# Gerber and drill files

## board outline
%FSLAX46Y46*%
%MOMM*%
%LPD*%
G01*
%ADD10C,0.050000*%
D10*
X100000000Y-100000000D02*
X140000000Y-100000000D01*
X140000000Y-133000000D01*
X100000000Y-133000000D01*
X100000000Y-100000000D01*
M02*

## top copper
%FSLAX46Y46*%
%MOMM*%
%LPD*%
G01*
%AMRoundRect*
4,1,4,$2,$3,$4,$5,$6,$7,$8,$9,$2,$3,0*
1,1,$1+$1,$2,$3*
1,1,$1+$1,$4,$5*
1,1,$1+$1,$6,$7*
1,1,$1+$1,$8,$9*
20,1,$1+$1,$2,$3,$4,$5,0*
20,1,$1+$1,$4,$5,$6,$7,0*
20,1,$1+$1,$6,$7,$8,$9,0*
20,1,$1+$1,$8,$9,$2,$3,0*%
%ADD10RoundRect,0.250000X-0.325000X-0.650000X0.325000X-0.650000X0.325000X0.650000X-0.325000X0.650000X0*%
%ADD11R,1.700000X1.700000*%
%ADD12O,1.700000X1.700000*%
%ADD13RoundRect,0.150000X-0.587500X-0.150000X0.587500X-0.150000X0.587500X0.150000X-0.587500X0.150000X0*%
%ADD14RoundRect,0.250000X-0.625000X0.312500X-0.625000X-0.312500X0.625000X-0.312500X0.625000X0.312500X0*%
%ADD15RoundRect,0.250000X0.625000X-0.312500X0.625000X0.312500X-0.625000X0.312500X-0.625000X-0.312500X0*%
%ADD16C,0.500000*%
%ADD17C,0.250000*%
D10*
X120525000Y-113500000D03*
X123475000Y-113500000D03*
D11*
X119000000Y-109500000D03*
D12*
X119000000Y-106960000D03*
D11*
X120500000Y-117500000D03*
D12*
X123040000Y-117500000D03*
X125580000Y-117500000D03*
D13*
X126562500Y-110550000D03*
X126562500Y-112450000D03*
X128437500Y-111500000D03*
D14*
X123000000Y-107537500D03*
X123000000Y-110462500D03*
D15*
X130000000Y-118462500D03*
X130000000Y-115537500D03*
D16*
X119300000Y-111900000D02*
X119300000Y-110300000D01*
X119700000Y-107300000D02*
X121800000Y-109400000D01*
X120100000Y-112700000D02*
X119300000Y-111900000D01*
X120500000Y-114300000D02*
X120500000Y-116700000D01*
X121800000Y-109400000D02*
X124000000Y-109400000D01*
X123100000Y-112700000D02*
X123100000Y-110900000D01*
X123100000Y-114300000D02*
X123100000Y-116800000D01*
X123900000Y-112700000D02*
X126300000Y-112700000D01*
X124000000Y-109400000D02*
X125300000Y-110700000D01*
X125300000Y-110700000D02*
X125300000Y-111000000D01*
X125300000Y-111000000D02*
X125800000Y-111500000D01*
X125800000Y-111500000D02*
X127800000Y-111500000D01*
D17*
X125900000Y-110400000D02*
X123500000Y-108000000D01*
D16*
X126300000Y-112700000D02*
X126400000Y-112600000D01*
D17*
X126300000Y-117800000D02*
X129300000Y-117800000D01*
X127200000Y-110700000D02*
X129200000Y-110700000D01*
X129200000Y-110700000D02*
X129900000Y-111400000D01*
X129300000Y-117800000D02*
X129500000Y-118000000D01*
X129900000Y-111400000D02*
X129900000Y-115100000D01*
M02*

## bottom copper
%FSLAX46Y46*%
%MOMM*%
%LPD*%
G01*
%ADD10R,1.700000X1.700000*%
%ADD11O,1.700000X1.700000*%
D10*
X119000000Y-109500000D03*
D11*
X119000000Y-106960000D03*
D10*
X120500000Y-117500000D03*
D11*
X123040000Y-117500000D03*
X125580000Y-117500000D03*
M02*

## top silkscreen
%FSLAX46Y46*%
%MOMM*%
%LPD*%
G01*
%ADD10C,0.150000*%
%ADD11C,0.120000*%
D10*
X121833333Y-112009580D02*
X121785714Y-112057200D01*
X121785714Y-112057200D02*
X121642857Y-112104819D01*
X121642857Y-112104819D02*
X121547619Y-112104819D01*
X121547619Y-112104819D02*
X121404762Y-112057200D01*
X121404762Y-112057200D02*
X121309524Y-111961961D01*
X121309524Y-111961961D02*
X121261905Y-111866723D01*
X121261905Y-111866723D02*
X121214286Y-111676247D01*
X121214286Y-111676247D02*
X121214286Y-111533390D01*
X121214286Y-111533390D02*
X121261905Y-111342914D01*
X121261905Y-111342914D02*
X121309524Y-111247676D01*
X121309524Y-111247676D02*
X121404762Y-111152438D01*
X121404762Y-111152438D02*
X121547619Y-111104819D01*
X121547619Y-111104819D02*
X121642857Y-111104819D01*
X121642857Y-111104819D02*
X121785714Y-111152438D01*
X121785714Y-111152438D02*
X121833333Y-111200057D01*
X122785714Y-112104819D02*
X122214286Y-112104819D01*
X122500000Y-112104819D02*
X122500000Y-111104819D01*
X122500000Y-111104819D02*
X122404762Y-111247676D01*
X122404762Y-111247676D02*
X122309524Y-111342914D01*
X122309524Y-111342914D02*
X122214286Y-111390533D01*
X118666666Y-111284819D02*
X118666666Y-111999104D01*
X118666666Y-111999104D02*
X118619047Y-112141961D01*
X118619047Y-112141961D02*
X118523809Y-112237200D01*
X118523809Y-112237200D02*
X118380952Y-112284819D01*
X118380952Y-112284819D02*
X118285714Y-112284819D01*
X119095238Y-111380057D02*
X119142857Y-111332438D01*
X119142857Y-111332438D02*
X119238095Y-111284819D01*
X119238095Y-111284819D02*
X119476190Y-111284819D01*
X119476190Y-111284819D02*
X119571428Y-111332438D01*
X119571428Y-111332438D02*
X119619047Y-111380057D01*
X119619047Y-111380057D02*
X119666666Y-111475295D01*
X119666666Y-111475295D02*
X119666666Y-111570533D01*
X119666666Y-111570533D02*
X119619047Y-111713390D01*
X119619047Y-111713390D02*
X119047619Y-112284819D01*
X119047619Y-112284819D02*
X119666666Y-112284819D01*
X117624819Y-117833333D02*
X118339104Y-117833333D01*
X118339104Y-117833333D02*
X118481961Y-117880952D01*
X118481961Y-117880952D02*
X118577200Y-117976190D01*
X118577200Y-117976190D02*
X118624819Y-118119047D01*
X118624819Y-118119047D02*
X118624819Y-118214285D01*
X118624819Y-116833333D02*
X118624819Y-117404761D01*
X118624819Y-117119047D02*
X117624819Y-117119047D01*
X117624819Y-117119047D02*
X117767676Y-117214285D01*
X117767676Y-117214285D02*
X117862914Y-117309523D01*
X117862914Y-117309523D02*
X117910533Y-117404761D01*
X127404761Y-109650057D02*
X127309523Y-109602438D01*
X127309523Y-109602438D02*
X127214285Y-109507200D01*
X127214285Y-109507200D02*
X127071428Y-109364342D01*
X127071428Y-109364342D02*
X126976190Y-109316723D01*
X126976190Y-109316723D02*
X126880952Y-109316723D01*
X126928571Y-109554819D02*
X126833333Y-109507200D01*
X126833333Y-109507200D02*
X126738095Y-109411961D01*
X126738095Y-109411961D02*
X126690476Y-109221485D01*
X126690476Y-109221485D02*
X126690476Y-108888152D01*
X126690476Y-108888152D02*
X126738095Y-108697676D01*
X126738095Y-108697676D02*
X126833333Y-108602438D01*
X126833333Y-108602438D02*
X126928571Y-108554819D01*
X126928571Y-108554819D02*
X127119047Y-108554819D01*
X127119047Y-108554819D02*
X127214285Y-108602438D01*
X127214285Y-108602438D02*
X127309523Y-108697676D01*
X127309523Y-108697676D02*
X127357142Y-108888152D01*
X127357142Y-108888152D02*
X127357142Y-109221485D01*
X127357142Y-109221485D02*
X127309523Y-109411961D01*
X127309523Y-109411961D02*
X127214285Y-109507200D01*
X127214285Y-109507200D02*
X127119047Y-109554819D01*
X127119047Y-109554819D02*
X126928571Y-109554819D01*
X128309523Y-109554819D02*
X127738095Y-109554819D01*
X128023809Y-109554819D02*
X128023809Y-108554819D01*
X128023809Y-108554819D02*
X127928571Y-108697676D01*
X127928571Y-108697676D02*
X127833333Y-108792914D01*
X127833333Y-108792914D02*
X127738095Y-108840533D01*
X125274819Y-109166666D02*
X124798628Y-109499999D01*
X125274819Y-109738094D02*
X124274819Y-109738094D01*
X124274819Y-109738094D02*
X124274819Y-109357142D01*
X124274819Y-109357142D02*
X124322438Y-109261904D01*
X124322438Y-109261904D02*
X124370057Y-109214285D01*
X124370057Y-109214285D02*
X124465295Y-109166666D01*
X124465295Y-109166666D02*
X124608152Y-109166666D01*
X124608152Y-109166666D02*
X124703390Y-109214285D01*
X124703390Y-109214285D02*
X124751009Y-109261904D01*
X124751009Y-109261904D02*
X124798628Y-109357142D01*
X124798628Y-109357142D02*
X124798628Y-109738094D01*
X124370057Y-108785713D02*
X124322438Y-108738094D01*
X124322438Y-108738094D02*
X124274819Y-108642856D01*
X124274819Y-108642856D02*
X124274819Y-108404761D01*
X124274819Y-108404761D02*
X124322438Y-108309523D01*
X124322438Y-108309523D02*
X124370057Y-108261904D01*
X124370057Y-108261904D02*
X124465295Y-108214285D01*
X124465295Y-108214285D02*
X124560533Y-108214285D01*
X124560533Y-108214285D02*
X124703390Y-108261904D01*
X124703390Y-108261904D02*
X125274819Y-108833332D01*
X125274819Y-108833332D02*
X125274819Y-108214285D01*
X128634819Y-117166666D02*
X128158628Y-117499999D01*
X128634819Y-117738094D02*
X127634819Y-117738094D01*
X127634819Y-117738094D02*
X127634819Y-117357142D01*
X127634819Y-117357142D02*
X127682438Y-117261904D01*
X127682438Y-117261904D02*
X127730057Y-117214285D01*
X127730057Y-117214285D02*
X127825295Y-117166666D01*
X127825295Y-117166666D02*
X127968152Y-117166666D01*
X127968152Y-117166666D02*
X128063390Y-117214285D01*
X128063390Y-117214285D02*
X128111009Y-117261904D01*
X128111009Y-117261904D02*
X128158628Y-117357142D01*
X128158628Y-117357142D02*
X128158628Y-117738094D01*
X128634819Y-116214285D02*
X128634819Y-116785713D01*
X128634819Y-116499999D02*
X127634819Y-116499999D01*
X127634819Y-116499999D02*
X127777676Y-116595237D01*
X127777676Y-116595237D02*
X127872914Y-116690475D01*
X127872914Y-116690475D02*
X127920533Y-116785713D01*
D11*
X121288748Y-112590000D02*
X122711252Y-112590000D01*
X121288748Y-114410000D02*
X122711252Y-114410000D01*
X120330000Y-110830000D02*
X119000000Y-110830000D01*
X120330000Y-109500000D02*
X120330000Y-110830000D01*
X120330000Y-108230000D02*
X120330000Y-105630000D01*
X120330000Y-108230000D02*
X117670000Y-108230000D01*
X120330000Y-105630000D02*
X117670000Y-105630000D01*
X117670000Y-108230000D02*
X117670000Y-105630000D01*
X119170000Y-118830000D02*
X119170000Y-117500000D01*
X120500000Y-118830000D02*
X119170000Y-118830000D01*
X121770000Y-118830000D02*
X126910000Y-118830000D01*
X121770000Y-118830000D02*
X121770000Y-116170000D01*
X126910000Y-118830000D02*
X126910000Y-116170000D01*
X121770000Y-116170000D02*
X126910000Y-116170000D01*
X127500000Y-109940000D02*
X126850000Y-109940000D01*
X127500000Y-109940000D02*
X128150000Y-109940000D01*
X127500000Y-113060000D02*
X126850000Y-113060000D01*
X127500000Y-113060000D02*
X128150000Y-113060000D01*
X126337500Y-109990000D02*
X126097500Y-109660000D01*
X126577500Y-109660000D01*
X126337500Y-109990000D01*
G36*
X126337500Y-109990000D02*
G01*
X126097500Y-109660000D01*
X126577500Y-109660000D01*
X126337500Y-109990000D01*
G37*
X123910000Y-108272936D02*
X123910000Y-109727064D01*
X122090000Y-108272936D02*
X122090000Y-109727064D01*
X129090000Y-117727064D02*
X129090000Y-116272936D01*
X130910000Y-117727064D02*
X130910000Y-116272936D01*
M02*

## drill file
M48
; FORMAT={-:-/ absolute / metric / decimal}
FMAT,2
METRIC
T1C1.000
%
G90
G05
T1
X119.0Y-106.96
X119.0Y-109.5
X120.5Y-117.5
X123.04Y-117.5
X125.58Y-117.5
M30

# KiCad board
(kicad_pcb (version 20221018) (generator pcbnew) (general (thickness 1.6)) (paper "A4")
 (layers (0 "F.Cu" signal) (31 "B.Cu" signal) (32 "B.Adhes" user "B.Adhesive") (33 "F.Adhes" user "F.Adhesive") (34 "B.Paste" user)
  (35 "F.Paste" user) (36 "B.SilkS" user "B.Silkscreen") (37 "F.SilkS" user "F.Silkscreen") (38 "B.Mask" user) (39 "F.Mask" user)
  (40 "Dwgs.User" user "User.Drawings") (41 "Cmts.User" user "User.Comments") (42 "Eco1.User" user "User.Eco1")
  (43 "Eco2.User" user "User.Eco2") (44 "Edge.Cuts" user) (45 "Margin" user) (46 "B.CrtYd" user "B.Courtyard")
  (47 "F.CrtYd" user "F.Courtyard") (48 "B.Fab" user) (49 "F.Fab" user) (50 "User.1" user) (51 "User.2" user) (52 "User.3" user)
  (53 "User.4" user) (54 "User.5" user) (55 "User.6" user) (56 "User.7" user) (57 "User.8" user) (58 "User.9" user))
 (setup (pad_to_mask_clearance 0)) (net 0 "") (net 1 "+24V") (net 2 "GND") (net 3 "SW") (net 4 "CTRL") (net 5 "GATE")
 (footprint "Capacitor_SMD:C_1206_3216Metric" (layer "F.Cu") (at 122 113.5)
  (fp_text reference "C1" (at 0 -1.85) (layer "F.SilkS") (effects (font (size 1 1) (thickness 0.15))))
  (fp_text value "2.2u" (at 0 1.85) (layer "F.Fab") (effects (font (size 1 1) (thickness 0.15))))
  (fp_line (start -0.711252 -0.91) (end 0.711252 -0.91) (stroke (width 0.12) (type solid)) (layer "F.SilkS"))
  (fp_line (start -0.711252 0.91) (end 0.711252 0.91) (stroke (width 0.12) (type solid)) (layer "F.SilkS"))
  (pad "1" smd roundrect (at -1.475 0) (size 1.15 1.8) (layers "F.Cu" "F.Paste" "F.Mask") (roundrect_rratio 0.217391) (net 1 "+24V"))
  (pad "2" smd roundrect (at 1.475 0) (size 1.15 1.8) (layers "F.Cu" "F.Paste" "F.Mask") (roundrect_rratio 0.217391) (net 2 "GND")))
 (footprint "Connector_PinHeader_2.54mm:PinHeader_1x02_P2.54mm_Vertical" (layer "F.Cu") (at 119 109.5 180)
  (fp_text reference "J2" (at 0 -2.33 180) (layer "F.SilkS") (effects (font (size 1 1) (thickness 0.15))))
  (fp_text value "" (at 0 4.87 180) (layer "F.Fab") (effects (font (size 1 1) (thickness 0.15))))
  (fp_line (start -1.33 -1.33) (end 0 -1.33) (stroke (width 0.12) (type solid)) (layer "F.SilkS"))
  (fp_line (start -1.33 0) (end -1.33 -1.33) (stroke (width 0.12) (type solid)) (layer "F.SilkS"))
  (fp_line (start -1.33 1.27) (end -1.33 3.87) (stroke (width 0.12) (type solid)) (layer "F.SilkS"))
  (fp_line (start -1.33 1.27) (end 1.33 1.27) (stroke (width 0.12) (type solid)) (layer "F.SilkS"))
  (fp_line (start -1.33 3.87) (end 1.33 3.87) (stroke (width 0.12) (type solid)) (layer "F.SilkS"))
  (fp_line (start 1.33 1.27) (end 1.33 3.87) (stroke (width 0.12) (type solid)) (layer "F.SilkS"))
  (pad "1" thru_hole rect (at 0 0 180) (size 1.7 1.7) (drill 1) (layers "*.Cu" "*.Mask") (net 1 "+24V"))
  (pad "2" thru_hole oval (at 0 2.54 180) (size 1.7 1.7) (drill 1) (layers "*.Cu" "*.Mask") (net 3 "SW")))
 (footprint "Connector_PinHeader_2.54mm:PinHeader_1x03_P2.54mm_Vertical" (layer "F.Cu") (at 120.5 117.5 90)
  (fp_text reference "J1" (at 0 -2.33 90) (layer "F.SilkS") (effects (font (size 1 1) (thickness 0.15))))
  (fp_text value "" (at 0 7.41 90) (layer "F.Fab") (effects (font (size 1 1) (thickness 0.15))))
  (fp_line (start -1.33 -1.33) (end 0 -1.33) (stroke (width 0.12) (type solid)) (layer "F.SilkS"))
  (fp_line (start -1.33 0) (end -1.33 -1.33) (stroke (width 0.12) (type solid)) (layer "F.SilkS"))
  (fp_line (start -1.33 1.27) (end -1.33 6.41) (stroke (width 0.12) (type solid)) (layer "F.SilkS"))
  (fp_line (start -1.33 1.27) (end 1.33 1.27) (stroke (width 0.12) (type solid)) (layer "F.SilkS"))
  (fp_line (start -1.33 6.41) (end 1.33 6.41) (stroke (width 0.12) (type solid)) (layer "F.SilkS"))
  (fp_line (start 1.33 1.27) (end 1.33 6.41) (stroke (width 0.12) (type solid)) (layer "F.SilkS"))
  (pad "1" thru_hole rect (at 0 0 90) (size 1.7 1.7) (drill 1) (layers "*.Cu" "*.Mask") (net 1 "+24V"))
  (pad "2" thru_hole oval (at 0 2.54 90) (size 1.7 1.7) (drill 1) (layers "*.Cu" "*.Mask") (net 2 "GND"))
  (pad "3" thru_hole oval (at 0 5.08 90) (size 1.7 1.7) (drill 1) (layers "*.Cu" "*.Mask") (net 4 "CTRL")))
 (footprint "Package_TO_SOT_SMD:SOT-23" (layer "F.Cu") (at 127.5 111.5)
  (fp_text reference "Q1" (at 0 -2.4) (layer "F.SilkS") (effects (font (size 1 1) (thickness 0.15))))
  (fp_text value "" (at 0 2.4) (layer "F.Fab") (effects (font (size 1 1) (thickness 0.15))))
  (fp_line (start 0 -1.56) (end -0.65 -1.56) (stroke (width 0.12) (type solid)) (layer "F.SilkS"))
  (fp_line (start 0 -1.56) (end 0.65 -1.56) (stroke (width 0.12) (type solid)) (layer "F.SilkS"))
  (fp_line (start 0 1.56) (end -0.65 1.56) (stroke (width 0.12) (type solid)) (layer "F.SilkS"))
  (fp_line (start 0 1.56) (end 0.65 1.56) (stroke (width 0.12) (type solid)) (layer "F.SilkS"))
  (fp_poly
   (pts (xy -1.1625 -1.51) (xy -1.4025 -1.84) (xy -0.9225 -1.84) (xy -1.1625 -1.51)) (stroke (width 0.12) (type solid)) (fill solid)
   (layer "F.SilkS"))
  (pad "1" smd roundrect (at -0.9375 -0.95) (size 1.475 0.6) (layers "F.Cu" "F.Paste" "F.Mask") (roundrect_rratio 0.25) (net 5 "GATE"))
  (pad "2" smd roundrect (at -0.9375 0.95) (size 1.475 0.6) (layers "F.Cu" "F.Paste" "F.Mask") (roundrect_rratio 0.25) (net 2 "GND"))
  (pad "3" smd roundrect (at 0.9375 0) (size 1.475 0.6) (layers "F.Cu" "F.Paste" "F.Mask") (roundrect_rratio 0.25) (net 3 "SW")))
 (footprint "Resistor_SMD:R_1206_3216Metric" (layer "F.Cu") (at 123 109 -90)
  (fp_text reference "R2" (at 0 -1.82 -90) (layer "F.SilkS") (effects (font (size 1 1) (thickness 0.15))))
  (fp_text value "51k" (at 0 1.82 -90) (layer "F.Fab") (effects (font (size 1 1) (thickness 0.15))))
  (fp_line (start -0.727064 -0.91) (end 0.727064 -0.91) (stroke (width 0.12) (type solid)) (layer "F.SilkS"))
  (fp_line (start -0.727064 0.91) (end 0.727064 0.91) (stroke (width 0.12) (type solid)) (layer "F.SilkS"))
  (pad "1" smd roundrect (at -1.4625 0 270) (size 1.125 1.75) (layers "F.Cu" "F.Paste" "F.Mask") (roundrect_rratio 0.222222) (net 5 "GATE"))
  (pad "2" smd roundrect (at 1.4625 0 270) (size 1.125 1.75) (layers "F.Cu" "F.Paste" "F.Mask") (roundrect_rratio 0.222222) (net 2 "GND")))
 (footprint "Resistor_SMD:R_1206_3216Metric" (layer "F.Cu") (at 130 117 90)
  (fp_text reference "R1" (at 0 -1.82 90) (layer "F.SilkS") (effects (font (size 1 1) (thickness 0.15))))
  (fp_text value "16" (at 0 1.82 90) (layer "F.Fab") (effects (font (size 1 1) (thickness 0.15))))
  (fp_line (start -0.727064 -0.91) (end 0.727064 -0.91) (stroke (width 0.12) (type solid)) (layer "F.SilkS"))
  (fp_line (start -0.727064 0.91) (end 0.727064 0.91) (stroke (width 0.12) (type solid)) (layer "F.SilkS"))
  (pad "1" smd roundrect (at -1.4625 0 90) (size 1.125 1.75) (layers "F.Cu" "F.Paste" "F.Mask") (roundrect_rratio 0.222222) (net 4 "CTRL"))
  (pad "2" smd roundrect (at 1.4625 0 90) (size 1.125 1.75) (layers "F.Cu" "F.Paste" "F.Mask") (roundrect_rratio 0.222222) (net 5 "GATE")))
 (gr_rect (start 100 100) (end 140 133) (stroke (width 0.05) (type default)) (fill none) (layer "Edge.Cuts"))
 (segment (start 119.3 111.9) (end 119.3 110.3) (width 0.5) (layer "F.Cu") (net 1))
 (segment (start 119.7 107.3) (end 121.8 109.4) (width 0.5) (layer "F.Cu") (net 3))
 (segment (start 120.1 112.7) (end 119.3 111.9) (width 0.5) (layer "F.Cu") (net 1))
 (segment (start 120.5 114.3) (end 120.5 116.7) (width 0.5) (layer "F.Cu") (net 1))
 (segment (start 121.8 109.4) (end 124 109.4) (width 0.5) (layer "F.Cu") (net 3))
 (segment (start 123.1 112.7) (end 123.1 110.9) (width 0.5) (layer "F.Cu") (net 2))
 (segment (start 123.1 114.3) (end 123.1 116.8) (width 0.5) (layer "F.Cu") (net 2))
 (segment (start 123.9 112.7) (end 126.3 112.7) (width 0.5) (layer "F.Cu") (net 2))
 (segment (start 124 109.4) (end 125.3 110.7) (width 0.5) (layer "F.Cu") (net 3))
 (segment (start 125.3 110.7) (end 125.3 111) (width 0.5) (layer "F.Cu") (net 3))
 (segment (start 125.3 111) (end 125.8 111.5) (width 0.5) (layer "F.Cu") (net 3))
 (segment (start 125.8 111.5) (end 127.8 111.5) (width 0.5) (layer "F.Cu") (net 3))
 (segment (start 125.9 110.4) (end 123.5 108) (width 0.25) (layer "F.Cu") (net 5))
 (segment (start 126.3 112.7) (end 126.4 112.6) (width 0.5) (layer "F.Cu") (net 2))
 (segment (start 126.3 117.8) (end 129.3 117.8) (width 0.25) (layer "F.Cu") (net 4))
 (segment (start 127.2 110.7) (end 129.2 110.7) (width 0.25) (layer "F.Cu") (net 5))
 (segment (start 129.2 110.7) (end 129.9 111.4) (width 0.25) (layer "F.Cu") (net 5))
 (segment (start 129.3 117.8) (end 129.5 118) (width 0.25) (layer "F.Cu") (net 4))
 (segment (start 129.9 111.4) (end 129.9 115.1) (width 0.25) (layer "F.Cu") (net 5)))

